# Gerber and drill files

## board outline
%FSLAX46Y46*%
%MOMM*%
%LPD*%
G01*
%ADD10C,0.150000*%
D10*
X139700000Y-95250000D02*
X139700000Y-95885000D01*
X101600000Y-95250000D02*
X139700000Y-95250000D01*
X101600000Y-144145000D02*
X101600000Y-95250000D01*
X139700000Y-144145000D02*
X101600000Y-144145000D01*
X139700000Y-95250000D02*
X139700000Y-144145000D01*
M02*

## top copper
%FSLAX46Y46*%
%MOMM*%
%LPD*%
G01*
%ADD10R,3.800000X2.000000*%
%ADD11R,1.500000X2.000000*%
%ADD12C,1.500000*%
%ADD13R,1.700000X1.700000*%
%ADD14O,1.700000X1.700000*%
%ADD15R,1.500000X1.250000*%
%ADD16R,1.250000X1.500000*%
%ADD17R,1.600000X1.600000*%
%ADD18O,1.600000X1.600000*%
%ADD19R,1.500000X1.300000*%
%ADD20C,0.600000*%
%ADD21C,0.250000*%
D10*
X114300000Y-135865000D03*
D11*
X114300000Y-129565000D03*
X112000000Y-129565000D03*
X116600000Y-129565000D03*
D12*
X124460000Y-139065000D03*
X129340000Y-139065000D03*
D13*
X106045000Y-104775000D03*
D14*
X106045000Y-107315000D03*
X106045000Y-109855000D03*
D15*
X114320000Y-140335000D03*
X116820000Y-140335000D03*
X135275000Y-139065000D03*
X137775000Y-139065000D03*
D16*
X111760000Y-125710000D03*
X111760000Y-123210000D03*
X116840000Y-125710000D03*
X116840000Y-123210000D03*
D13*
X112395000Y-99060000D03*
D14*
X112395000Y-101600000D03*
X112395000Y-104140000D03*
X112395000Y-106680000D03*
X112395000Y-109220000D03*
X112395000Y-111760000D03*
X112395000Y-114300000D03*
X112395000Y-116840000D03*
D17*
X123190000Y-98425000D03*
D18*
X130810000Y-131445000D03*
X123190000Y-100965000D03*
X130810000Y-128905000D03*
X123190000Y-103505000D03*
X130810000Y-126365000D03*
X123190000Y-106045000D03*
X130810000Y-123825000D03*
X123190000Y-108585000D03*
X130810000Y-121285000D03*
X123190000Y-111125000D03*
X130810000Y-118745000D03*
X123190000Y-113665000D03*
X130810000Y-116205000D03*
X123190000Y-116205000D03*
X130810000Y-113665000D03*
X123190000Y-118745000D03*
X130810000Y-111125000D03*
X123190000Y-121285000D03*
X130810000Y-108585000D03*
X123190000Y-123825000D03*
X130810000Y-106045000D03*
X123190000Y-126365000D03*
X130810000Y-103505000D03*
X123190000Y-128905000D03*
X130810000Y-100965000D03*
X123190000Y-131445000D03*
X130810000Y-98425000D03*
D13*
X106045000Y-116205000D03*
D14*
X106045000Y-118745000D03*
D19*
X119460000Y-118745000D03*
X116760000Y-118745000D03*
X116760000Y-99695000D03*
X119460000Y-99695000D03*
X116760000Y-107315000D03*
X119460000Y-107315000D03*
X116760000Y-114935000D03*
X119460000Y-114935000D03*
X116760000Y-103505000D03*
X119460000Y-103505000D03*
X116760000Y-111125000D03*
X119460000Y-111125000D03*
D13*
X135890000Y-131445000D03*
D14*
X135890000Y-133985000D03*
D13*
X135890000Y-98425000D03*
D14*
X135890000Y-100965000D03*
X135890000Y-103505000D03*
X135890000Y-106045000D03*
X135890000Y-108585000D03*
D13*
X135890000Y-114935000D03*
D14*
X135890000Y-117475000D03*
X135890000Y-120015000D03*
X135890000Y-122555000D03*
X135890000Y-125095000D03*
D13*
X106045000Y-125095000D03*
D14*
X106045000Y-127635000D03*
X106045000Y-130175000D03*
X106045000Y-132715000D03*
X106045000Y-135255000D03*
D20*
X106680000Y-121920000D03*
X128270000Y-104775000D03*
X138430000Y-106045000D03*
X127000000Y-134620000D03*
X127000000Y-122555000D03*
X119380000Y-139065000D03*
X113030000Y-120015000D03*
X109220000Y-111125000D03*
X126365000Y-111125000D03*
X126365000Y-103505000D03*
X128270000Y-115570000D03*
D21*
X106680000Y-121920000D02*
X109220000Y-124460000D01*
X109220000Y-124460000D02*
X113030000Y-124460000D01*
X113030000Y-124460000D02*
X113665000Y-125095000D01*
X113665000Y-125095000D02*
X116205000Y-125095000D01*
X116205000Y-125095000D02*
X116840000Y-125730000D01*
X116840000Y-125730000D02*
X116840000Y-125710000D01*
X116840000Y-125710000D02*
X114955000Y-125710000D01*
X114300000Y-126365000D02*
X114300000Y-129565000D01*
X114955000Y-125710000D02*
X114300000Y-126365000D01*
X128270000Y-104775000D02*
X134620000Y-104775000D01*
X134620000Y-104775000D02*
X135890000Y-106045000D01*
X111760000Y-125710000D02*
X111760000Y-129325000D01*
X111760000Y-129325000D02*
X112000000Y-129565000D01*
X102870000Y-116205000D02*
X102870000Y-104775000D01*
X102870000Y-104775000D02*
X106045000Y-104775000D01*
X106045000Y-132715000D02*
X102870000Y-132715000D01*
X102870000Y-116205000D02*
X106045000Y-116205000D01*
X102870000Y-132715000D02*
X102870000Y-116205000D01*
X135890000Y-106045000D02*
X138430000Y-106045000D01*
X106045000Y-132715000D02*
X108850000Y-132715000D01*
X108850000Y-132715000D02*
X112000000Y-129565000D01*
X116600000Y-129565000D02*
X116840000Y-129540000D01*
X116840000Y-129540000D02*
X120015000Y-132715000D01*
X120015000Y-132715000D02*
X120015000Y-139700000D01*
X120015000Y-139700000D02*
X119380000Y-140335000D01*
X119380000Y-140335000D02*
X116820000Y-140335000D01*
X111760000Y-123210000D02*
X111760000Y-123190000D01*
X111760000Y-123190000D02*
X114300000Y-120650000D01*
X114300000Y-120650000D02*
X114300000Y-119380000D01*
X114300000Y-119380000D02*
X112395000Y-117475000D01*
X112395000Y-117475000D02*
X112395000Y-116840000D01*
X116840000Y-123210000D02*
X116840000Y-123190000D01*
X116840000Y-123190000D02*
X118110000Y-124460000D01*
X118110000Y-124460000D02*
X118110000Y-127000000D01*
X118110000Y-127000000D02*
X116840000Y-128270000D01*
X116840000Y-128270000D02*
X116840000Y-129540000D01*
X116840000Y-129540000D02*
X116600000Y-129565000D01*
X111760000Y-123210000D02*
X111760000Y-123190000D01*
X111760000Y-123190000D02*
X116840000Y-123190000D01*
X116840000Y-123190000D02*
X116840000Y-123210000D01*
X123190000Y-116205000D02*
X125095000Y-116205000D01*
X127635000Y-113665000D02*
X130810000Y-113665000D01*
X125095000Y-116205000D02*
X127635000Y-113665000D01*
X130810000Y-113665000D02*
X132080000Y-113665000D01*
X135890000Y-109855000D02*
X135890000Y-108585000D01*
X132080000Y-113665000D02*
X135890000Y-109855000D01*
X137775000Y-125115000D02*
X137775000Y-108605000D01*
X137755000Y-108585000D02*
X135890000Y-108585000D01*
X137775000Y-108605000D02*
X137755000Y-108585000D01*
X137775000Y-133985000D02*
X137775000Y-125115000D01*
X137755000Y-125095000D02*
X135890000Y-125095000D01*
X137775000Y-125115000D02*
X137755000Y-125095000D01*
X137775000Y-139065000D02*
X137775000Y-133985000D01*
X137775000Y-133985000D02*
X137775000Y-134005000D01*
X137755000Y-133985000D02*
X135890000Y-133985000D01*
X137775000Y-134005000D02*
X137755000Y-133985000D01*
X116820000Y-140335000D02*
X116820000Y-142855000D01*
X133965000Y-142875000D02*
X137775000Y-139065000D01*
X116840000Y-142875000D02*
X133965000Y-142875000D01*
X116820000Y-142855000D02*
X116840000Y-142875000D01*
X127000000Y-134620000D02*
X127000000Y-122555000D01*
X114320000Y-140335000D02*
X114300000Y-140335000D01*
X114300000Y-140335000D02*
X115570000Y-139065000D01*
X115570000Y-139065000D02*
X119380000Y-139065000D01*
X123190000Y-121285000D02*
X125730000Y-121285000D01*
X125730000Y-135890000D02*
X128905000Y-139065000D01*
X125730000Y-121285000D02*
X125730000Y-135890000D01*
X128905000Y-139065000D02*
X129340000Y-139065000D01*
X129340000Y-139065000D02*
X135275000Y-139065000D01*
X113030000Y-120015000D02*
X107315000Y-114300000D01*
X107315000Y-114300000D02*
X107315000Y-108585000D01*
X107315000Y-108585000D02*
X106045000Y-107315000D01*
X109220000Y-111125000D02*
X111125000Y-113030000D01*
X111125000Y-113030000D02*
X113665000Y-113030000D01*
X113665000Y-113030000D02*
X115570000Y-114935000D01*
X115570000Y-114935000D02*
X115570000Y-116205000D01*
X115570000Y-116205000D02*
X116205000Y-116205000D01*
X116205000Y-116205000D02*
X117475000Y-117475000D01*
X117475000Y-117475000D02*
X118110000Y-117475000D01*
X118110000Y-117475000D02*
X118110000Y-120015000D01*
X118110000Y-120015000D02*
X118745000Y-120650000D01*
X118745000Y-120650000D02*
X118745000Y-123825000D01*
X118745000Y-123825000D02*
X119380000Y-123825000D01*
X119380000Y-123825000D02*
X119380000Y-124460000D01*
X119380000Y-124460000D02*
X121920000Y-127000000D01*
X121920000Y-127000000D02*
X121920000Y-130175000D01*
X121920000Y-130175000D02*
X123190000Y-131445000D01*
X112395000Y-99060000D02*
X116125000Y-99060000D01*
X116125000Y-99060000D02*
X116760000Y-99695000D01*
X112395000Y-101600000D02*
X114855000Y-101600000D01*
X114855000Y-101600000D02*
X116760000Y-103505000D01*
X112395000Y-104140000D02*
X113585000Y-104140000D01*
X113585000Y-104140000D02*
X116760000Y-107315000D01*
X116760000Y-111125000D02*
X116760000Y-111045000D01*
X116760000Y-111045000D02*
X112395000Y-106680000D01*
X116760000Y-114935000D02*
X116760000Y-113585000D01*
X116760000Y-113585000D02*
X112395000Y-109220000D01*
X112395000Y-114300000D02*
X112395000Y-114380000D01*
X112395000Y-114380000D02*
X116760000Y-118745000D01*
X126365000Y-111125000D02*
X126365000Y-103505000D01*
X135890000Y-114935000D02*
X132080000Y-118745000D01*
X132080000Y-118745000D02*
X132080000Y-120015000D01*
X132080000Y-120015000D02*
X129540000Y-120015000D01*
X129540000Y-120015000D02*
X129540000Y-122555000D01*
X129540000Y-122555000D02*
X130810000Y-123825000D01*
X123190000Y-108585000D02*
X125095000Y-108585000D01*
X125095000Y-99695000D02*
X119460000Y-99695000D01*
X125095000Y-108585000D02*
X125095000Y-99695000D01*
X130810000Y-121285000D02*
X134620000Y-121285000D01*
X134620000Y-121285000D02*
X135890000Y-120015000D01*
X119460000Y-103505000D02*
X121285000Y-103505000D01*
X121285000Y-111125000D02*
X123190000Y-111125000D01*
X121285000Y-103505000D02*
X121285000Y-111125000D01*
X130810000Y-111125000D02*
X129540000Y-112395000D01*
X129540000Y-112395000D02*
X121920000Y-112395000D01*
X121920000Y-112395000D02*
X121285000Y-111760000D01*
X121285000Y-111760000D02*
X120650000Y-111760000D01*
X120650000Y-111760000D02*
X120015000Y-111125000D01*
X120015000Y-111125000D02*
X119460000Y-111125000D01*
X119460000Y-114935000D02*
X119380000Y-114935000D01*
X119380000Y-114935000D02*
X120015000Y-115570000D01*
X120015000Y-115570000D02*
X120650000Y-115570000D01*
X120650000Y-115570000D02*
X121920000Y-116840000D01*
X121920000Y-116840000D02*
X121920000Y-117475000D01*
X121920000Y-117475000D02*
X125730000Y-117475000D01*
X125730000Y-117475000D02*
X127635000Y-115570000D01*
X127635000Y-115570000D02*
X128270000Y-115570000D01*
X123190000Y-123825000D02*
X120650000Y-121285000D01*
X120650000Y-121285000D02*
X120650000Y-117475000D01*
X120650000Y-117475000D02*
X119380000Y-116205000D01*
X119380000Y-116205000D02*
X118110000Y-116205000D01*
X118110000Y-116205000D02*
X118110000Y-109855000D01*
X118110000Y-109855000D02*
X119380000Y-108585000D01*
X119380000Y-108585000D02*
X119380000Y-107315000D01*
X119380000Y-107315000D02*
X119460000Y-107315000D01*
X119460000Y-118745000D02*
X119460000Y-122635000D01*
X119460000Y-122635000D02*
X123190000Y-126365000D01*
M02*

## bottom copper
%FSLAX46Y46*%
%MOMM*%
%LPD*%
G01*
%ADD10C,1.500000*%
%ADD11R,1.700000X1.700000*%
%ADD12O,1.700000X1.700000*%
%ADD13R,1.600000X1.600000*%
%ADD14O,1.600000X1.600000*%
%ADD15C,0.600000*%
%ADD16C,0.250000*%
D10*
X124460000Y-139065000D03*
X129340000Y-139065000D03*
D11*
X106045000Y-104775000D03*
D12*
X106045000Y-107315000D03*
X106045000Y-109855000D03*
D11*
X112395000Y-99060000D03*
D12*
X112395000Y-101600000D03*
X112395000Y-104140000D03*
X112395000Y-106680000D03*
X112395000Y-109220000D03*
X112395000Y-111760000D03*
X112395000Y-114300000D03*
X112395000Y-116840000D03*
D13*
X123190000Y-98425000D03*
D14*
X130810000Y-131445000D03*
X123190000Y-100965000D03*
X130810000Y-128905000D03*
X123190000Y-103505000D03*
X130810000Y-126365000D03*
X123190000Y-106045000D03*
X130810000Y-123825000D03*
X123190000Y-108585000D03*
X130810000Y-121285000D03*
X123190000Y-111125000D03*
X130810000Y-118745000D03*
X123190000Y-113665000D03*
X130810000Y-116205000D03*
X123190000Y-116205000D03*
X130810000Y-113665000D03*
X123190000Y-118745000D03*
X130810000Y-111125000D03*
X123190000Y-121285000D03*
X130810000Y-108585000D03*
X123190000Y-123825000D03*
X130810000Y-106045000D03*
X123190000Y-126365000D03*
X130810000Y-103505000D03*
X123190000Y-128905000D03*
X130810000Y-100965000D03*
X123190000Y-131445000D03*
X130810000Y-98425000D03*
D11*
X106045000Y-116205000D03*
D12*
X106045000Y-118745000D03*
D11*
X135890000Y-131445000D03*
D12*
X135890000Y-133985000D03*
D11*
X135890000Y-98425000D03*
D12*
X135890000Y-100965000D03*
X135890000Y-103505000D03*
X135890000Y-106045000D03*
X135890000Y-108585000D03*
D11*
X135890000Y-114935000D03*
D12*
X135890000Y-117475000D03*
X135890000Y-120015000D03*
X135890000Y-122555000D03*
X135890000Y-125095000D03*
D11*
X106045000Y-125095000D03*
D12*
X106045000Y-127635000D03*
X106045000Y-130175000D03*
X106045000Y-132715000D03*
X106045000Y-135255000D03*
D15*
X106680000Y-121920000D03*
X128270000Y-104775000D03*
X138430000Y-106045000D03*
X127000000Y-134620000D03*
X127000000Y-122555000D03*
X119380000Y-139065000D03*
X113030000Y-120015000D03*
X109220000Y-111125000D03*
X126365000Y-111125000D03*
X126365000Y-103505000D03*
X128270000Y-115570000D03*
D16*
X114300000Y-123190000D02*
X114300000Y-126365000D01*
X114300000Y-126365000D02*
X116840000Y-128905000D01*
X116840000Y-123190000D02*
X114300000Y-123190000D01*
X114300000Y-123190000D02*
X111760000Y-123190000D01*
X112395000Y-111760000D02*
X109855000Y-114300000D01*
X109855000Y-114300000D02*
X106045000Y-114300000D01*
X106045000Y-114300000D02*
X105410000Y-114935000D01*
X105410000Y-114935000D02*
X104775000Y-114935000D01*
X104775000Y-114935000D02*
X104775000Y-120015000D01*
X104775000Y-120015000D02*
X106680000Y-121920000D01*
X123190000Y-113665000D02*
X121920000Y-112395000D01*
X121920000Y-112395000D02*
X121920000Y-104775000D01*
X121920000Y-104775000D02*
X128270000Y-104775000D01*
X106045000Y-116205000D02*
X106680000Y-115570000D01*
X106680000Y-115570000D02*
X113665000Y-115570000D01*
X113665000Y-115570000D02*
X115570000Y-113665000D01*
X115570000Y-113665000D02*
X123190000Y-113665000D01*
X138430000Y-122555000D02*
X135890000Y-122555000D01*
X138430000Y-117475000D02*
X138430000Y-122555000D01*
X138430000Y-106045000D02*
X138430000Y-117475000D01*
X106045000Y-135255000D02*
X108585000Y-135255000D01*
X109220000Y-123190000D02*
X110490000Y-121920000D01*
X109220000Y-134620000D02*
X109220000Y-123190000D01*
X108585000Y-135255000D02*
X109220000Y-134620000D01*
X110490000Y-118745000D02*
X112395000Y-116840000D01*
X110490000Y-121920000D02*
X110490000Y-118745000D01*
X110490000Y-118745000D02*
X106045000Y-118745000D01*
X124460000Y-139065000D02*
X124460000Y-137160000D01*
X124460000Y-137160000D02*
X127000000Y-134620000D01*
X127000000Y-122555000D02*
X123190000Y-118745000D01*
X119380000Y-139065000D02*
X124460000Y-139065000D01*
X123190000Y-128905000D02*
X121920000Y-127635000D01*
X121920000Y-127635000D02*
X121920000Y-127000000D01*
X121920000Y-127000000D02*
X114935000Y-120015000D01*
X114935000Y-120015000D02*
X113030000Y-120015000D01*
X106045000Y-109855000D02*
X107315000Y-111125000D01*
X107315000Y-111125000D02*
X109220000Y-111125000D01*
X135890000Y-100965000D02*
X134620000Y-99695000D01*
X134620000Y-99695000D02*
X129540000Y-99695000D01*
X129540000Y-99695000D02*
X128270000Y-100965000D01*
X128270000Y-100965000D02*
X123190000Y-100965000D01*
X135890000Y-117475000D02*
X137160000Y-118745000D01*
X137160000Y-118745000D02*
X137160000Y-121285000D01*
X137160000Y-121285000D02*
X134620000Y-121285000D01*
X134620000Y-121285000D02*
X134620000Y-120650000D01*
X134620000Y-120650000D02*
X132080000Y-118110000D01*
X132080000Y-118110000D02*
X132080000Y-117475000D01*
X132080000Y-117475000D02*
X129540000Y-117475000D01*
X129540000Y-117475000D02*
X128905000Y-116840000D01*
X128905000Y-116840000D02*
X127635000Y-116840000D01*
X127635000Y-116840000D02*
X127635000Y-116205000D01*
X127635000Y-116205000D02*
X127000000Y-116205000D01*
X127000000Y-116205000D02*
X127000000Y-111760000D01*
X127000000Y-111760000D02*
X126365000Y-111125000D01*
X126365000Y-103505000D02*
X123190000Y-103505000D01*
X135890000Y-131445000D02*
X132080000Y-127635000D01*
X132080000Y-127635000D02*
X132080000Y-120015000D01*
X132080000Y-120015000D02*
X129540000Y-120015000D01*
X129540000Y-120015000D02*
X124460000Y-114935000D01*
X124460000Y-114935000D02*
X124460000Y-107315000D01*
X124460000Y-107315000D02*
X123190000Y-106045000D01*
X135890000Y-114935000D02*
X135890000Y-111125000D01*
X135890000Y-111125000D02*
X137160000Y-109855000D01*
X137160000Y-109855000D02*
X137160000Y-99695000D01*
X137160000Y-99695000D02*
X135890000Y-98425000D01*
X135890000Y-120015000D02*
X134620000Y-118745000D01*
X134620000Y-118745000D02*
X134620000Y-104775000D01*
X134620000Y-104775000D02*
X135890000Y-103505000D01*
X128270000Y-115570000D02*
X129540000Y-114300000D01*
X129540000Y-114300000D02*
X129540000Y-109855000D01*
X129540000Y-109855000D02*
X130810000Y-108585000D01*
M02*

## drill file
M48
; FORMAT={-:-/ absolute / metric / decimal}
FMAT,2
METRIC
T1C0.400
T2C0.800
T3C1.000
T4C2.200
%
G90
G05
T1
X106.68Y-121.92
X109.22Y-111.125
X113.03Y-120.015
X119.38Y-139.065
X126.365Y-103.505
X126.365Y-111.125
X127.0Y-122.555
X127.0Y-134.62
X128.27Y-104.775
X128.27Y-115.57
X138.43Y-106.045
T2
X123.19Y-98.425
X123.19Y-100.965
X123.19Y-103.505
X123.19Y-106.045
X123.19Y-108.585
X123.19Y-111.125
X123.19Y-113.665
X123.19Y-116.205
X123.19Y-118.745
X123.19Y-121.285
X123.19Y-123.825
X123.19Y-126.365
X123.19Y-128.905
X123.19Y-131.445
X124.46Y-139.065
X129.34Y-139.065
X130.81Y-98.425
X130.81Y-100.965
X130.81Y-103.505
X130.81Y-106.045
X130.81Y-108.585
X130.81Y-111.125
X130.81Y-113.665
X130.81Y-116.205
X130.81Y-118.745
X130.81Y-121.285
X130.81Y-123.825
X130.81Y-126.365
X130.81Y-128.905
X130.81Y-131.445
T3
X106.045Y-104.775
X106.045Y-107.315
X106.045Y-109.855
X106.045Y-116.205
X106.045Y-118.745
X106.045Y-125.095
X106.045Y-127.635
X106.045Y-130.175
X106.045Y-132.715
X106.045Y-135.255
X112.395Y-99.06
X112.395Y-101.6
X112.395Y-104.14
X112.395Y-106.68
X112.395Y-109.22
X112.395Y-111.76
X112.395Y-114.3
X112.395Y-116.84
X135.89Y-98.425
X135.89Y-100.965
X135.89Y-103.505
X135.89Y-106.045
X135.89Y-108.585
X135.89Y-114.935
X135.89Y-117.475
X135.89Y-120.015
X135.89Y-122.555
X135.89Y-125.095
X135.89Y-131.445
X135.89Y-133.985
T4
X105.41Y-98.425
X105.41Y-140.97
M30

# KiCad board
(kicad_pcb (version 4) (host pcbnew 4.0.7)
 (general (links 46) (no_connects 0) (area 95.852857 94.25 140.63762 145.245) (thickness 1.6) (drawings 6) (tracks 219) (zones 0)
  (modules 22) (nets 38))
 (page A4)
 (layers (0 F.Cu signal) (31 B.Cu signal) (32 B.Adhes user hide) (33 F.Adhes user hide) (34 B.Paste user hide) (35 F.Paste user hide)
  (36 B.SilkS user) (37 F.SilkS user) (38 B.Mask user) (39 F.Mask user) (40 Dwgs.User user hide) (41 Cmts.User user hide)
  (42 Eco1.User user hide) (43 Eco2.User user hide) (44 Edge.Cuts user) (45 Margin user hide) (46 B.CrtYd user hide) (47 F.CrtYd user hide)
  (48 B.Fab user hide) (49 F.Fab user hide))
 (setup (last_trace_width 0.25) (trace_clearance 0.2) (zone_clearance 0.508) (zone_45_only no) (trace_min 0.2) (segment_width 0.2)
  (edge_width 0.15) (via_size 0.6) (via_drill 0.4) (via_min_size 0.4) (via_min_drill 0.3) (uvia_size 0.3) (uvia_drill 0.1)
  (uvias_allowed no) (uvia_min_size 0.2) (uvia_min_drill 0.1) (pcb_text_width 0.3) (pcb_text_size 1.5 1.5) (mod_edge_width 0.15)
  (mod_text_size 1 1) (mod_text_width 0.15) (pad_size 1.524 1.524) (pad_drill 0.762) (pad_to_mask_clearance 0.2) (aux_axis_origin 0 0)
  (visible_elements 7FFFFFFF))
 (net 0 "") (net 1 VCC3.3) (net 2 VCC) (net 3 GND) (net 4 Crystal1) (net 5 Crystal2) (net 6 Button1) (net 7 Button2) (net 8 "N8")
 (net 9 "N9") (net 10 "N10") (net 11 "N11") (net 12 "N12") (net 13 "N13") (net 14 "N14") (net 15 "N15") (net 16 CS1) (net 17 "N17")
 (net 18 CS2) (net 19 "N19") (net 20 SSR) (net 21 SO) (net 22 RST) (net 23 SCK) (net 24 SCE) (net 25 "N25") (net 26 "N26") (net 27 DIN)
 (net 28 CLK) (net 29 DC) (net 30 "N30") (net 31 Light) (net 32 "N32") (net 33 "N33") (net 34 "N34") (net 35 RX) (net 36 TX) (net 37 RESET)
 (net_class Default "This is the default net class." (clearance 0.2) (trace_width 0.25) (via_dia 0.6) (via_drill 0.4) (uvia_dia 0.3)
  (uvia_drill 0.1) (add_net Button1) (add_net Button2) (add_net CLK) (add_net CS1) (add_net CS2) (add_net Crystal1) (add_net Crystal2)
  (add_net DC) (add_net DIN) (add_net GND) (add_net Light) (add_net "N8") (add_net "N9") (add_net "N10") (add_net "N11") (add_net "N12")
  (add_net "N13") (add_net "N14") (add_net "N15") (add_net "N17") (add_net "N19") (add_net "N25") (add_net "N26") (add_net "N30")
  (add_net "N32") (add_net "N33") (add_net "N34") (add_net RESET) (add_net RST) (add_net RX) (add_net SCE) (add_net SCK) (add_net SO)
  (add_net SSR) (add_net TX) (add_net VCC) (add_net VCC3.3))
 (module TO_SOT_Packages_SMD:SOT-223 (layer F.Cu) (at 114.3 132.715 270)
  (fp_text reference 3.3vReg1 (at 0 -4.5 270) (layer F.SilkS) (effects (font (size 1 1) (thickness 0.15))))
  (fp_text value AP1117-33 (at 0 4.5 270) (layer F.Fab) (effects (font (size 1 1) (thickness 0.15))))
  (pad 4 smd rect (at 3.15 0 270) (size 2 3.8) (layers F.Cu F.Paste F.Mask))
  (pad 2 smd rect (at -3.15 0 270) (size 2 1.5) (layers F.Cu F.Paste F.Mask) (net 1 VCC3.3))
  (pad 3 smd rect (at -3.15 2.3 270) (size 2 1.5) (layers F.Cu F.Paste F.Mask) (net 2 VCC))
  (pad 1 smd rect (at -3.15 -2.3 270) (size 2 1.5) (layers F.Cu F.Paste F.Mask) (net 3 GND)))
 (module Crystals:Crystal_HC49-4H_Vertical (layer F.Cu) (at 124.46 139.065)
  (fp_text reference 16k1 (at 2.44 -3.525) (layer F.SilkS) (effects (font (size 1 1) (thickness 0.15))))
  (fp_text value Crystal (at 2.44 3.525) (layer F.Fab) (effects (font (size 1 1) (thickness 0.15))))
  (pad 1 thru_hole circle (at 0 0) (size 1.5 1.5) (drill 0.8) (layers *.Cu *.Mask) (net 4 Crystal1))
  (pad 2 thru_hole circle (at 4.88 0) (size 1.5 1.5) (drill 0.8) (layers *.Cu *.Mask) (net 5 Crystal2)))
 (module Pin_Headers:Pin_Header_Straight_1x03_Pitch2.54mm (layer F.Cu) (at 106.045 104.775)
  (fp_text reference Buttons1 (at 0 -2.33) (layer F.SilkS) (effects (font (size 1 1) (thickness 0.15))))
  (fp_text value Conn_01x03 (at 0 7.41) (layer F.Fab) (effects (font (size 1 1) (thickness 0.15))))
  (pad 1 thru_hole rect (at 0 0) (size 1.7 1.7) (drill 1) (layers *.Cu *.Mask) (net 2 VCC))
  (pad 2 thru_hole oval (at 0 2.54) (size 1.7 1.7) (drill 1) (layers *.Cu *.Mask) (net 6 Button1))
  (pad 3 thru_hole oval (at 0 5.08) (size 1.7 1.7) (drill 1) (layers *.Cu *.Mask) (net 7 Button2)))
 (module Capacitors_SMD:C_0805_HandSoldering (layer F.Cu) (at 115.57 140.335)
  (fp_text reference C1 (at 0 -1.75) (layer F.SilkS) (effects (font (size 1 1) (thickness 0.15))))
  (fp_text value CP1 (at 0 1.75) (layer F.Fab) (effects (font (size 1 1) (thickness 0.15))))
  (pad 1 smd rect (at -1.25 0) (size 1.5 1.25) (layers F.Cu F.Paste F.Mask) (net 4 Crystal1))
  (pad 2 smd rect (at 1.25 0) (size 1.5 1.25) (layers F.Cu F.Paste F.Mask) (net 3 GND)))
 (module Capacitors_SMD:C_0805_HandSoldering (layer F.Cu) (at 136.525 139.065)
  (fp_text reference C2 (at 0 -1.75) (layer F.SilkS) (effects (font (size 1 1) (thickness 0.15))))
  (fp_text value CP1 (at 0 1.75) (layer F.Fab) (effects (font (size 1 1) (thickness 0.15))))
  (pad 1 smd rect (at -1.25 0) (size 1.5 1.25) (layers F.Cu F.Paste F.Mask) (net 5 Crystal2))
  (pad 2 smd rect (at 1.25 0) (size 1.5 1.25) (layers F.Cu F.Paste F.Mask) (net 3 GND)))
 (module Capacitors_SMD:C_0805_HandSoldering (layer F.Cu) (at 111.76 124.46 90)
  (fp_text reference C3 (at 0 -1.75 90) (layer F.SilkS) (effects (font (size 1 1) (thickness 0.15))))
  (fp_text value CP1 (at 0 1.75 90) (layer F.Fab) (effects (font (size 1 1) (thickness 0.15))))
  (pad 1 smd rect (at -1.25 0 90) (size 1.5 1.25) (layers F.Cu F.Paste F.Mask) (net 2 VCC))
  (pad 2 smd rect (at 1.25 0 90) (size 1.5 1.25) (layers F.Cu F.Paste F.Mask) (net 3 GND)))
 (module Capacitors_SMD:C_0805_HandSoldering (layer F.Cu) (at 116.84 124.46 90)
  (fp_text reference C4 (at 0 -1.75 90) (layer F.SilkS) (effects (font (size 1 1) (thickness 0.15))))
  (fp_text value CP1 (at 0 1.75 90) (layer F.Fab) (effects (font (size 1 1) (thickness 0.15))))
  (pad 1 smd rect (at -1.25 0 90) (size 1.5 1.25) (layers F.Cu F.Paste F.Mask) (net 1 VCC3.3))
  (pad 2 smd rect (at 1.25 0 90) (size 1.5 1.25) (layers F.Cu F.Paste F.Mask) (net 3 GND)))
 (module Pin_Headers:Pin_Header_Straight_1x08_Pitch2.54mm (layer F.Cu) (at 112.395 99.06)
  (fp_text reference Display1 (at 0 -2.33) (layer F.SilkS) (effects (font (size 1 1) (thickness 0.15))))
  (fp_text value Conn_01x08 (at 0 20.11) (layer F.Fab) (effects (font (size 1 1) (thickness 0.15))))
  (pad 1 thru_hole rect (at 0 0) (size 1.7 1.7) (drill 1) (layers *.Cu *.Mask) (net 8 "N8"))
  (pad 2 thru_hole oval (at 0 2.54) (size 1.7 1.7) (drill 1) (layers *.Cu *.Mask) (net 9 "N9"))
  (pad 3 thru_hole oval (at 0 5.08) (size 1.7 1.7) (drill 1) (layers *.Cu *.Mask) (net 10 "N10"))
  (pad 4 thru_hole oval (at 0 7.62) (size 1.7 1.7) (drill 1) (layers *.Cu *.Mask) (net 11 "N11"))
  (pad 5 thru_hole oval (at 0 10.16) (size 1.7 1.7) (drill 1) (layers *.Cu *.Mask) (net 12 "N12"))
  (pad 6 thru_hole oval (at 0 12.7) (size 1.7 1.7) (drill 1) (layers *.Cu *.Mask) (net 1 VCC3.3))
  (pad 7 thru_hole oval (at 0 15.24) (size 1.7 1.7) (drill 1) (layers *.Cu *.Mask) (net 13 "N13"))
  (pad 8 thru_hole oval (at 0 17.78) (size 1.7 1.7) (drill 1) (layers *.Cu *.Mask) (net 3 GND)))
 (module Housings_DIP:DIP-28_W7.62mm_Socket (layer F.Cu) (at 123.19 98.425)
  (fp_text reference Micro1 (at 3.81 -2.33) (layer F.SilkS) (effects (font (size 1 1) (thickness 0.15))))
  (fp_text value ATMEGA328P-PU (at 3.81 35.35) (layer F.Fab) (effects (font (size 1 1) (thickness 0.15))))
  (pad 1 thru_hole rect (at 0 0) (size 1.6 1.6) (drill 0.8) (layers *.Cu *.Mask) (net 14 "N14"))
  (pad 15 thru_hole oval (at 7.62 33.02) (size 1.6 1.6) (drill 0.8) (layers *.Cu *.Mask) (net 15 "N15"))
  (pad 2 thru_hole oval (at 0 2.54) (size 1.6 1.6) (drill 0.8) (layers *.Cu *.Mask) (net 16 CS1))
  (pad 16 thru_hole oval (at 7.62 30.48) (size 1.6 1.6) (drill 0.8) (layers *.Cu *.Mask) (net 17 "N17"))
  (pad 3 thru_hole oval (at 0 5.08) (size 1.6 1.6) (drill 0.8) (layers *.Cu *.Mask) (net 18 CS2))
  (pad 17 thru_hole oval (at 7.62 27.94) (size 1.6 1.6) (drill 0.8) (layers *.Cu *.Mask) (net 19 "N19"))
  (pad 4 thru_hole oval (at 0 7.62) (size 1.6 1.6) (drill 0.8) (layers *.Cu *.Mask) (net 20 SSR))
  (pad 18 thru_hole oval (at 7.62 25.4) (size 1.6 1.6) (drill 0.8) (layers *.Cu *.Mask) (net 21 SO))
  (pad 5 thru_hole oval (at 0 10.16) (size 1.6 1.6) (drill 0.8) (layers *.Cu *.Mask) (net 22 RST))
  (pad 19 thru_hole oval (at 7.62 22.86) (size 1.6 1.6) (drill 0.8) (layers *.Cu *.Mask) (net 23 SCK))
  (pad 6 thru_hole oval (at 0 12.7) (size 1.6 1.6) (drill 0.8) (layers *.Cu *.Mask) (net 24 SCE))
  (pad 20 thru_hole oval (at 7.62 20.32) (size 1.6 1.6) (drill 0.8) (layers *.Cu *.Mask) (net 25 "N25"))
  (pad 7 thru_hole oval (at 0 15.24) (size 1.6 1.6) (drill 0.8) (layers *.Cu *.Mask) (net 2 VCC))
  (pad 21 thru_hole oval (at 7.62 17.78) (size 1.6 1.6) (drill 0.8) (layers *.Cu *.Mask) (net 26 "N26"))
  (pad 8 thru_hole oval (at 0 17.78) (size 1.6 1.6) (drill 0.8) (layers *.Cu *.Mask) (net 3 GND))
  (pad 22 thru_hole oval (at 7.62 15.24) (size 1.6 1.6) (drill 0.8) (layers *.Cu *.Mask) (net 3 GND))
  (pad 9 thru_hole oval (at 0 20.32) (size 1.6 1.6) (drill 0.8) (layers *.Cu *.Mask) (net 4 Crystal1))
  (pad 23 thru_hole oval (at 7.62 12.7) (size 1.6 1.6) (drill 0.8) (layers *.Cu *.Mask) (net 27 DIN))
  (pad 10 thru_hole oval (at 0 22.86) (size 1.6 1.6) (drill 0.8) (layers *.Cu *.Mask) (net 5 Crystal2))
  (pad 24 thru_hole oval (at 7.62 10.16) (size 1.6 1.6) (drill 0.8) (layers *.Cu *.Mask) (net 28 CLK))
  (pad 11 thru_hole oval (at 0 25.4) (size 1.6 1.6) (drill 0.8) (layers *.Cu *.Mask) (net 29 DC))
  (pad 25 thru_hole oval (at 7.62 7.62) (size 1.6 1.6) (drill 0.8) (layers *.Cu *.Mask) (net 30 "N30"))
  (pad 12 thru_hole oval (at 0 27.94) (size 1.6 1.6) (drill 0.8) (layers *.Cu *.Mask) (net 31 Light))
  (pad 26 thru_hole oval (at 7.62 5.08) (size 1.6 1.6) (drill 0.8) (layers *.Cu *.Mask) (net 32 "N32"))
  (pad 13 thru_hole oval (at 0 30.48) (size 1.6 1.6) (drill 0.8) (layers *.Cu *.Mask) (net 6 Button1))
  (pad 27 thru_hole oval (at 7.62 2.54) (size 1.6 1.6) (drill 0.8) (layers *.Cu *.Mask) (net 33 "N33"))
  (pad 14 thru_hole oval (at 0 33.02) (size 1.6 1.6) (drill 0.8) (layers *.Cu *.Mask) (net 7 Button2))
  (pad 28 thru_hole oval (at 7.62 0) (size 1.6 1.6) (drill 0.8) (layers *.Cu *.Mask) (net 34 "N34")))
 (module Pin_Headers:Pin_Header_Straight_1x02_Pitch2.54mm (layer F.Cu) (at 106.045 116.205)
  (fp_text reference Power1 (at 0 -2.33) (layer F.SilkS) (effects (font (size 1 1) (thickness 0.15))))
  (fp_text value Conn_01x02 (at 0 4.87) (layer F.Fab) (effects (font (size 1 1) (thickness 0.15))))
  (pad 1 thru_hole rect (at 0 0) (size 1.7 1.7) (drill 1) (layers *.Cu *.Mask) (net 2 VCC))
  (pad 2 thru_hole oval (at 0 2.54) (size 1.7 1.7) (drill 1) (layers *.Cu *.Mask) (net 3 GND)))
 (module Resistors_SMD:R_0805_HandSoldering (layer F.Cu) (at 118.11 118.745 180)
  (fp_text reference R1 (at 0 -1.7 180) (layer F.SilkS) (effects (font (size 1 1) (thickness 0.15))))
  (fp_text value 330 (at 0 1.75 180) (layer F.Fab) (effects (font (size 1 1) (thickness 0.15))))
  (pad 1 smd rect (at -1.35 0 180) (size 1.5 1.3) (layers F.Cu F.Paste F.Mask) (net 31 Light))
  (pad 2 smd rect (at 1.35 0 180) (size 1.5 1.3) (layers F.Cu F.Paste F.Mask) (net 13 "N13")))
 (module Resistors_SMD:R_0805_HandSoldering (layer F.Cu) (at 118.11 99.695)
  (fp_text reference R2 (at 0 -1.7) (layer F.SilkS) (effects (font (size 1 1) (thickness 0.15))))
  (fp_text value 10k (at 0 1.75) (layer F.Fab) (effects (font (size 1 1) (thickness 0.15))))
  (pad 1 smd rect (at -1.35 0) (size 1.5 1.3) (layers F.Cu F.Paste F.Mask) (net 8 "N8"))
  (pad 2 smd rect (at 1.35 0) (size 1.5 1.3) (layers F.Cu F.Paste F.Mask) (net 22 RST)))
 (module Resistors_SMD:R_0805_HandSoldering (layer F.Cu) (at 118.11 107.315)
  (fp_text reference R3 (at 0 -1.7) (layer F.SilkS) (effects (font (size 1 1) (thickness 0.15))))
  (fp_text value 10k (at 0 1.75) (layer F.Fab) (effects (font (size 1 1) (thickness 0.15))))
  (pad 1 smd rect (at -1.35 0) (size 1.5 1.3) (layers F.Cu F.Paste F.Mask) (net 10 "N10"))
  (pad 2 smd rect (at 1.35 0) (size 1.5 1.3) (layers F.Cu F.Paste F.Mask) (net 29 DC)))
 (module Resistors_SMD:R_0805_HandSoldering (layer F.Cu) (at 118.11 114.935)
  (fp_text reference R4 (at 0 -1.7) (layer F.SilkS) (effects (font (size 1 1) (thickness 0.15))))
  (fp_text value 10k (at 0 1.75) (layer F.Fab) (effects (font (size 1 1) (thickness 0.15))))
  (pad 1 smd rect (at -1.35 0) (size 1.5 1.3) (layers F.Cu F.Paste F.Mask) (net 12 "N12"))
  (pad 2 smd rect (at 1.35 0) (size 1.5 1.3) (layers F.Cu F.Paste F.Mask) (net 28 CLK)))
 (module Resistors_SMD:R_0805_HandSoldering (layer F.Cu) (at 118.11 103.505)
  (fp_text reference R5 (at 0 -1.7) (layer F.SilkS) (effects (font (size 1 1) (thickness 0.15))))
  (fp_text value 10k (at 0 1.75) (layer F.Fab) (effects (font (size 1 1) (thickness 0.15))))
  (pad 1 smd rect (at -1.35 0) (size 1.5 1.3) (layers F.Cu F.Paste F.Mask) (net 9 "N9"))
  (pad 2 smd rect (at 1.35 0) (size 1.5 1.3) (layers F.Cu F.Paste F.Mask) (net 24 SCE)))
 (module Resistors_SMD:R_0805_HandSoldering (layer F.Cu) (at 118.11 111.125)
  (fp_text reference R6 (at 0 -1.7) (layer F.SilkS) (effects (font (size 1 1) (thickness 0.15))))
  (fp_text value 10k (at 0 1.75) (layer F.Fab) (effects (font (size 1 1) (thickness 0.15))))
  (pad 1 smd rect (at -1.35 0) (size 1.5 1.3) (layers F.Cu F.Paste F.Mask) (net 11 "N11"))
  (pad 2 smd rect (at 1.35 0) (size 1.5 1.3) (layers F.Cu F.Paste F.Mask) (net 27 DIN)))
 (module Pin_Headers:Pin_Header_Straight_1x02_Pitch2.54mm (layer F.Cu) (at 135.89 131.445)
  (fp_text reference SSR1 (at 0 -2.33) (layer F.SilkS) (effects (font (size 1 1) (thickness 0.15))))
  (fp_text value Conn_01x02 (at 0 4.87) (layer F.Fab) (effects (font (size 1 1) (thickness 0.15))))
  (pad 1 thru_hole rect (at 0 0) (size 1.7 1.7) (drill 1) (layers *.Cu *.Mask) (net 20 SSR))
  (pad 2 thru_hole oval (at 0 2.54) (size 1.7 1.7) (drill 1) (layers *.Cu *.Mask) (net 3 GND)))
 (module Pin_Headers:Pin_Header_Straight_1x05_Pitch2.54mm (layer F.Cu) (at 135.89 98.425)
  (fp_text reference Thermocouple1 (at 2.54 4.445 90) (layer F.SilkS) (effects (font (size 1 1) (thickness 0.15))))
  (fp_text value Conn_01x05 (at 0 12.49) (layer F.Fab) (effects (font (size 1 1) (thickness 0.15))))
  (pad 1 thru_hole rect (at 0 0) (size 1.7 1.7) (drill 1) (layers *.Cu *.Mask) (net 21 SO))
  (pad 2 thru_hole oval (at 0 2.54) (size 1.7 1.7) (drill 1) (layers *.Cu *.Mask) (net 16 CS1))
  (pad 3 thru_hole oval (at 0 5.08) (size 1.7 1.7) (drill 1) (layers *.Cu *.Mask) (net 23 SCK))
  (pad 4 thru_hole oval (at 0 7.62) (size 1.7 1.7) (drill 1) (layers *.Cu *.Mask) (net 2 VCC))
  (pad 5 thru_hole oval (at 0 10.16) (size 1.7 1.7) (drill 1) (layers *.Cu *.Mask) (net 3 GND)))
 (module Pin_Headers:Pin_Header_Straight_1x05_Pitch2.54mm (layer F.Cu) (at 135.89 114.935)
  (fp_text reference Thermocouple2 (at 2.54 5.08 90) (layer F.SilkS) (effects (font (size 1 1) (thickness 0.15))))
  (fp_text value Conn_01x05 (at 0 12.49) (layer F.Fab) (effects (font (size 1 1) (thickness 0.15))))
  (pad 1 thru_hole rect (at 0 0) (size 1.7 1.7) (drill 1) (layers *.Cu *.Mask) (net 21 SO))
  (pad 2 thru_hole oval (at 0 2.54) (size 1.7 1.7) (drill 1) (layers *.Cu *.Mask) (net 18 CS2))
  (pad 3 thru_hole oval (at 0 5.08) (size 1.7 1.7) (drill 1) (layers *.Cu *.Mask) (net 23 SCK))
  (pad 4 thru_hole oval (at 0 7.62) (size 1.7 1.7) (drill 1) (layers *.Cu *.Mask) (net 2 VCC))
  (pad 5 thru_hole oval (at 0 10.16) (size 1.7 1.7) (drill 1) (layers *.Cu *.Mask) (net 3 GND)))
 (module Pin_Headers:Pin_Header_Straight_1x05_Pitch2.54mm (layer F.Cu) (at 106.045 125.095)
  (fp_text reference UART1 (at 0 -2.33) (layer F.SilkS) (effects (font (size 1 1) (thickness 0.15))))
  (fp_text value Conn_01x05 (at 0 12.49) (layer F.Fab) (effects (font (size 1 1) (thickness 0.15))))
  (pad 1 thru_hole rect (at 0 0) (size 1.7 1.7) (drill 1) (layers *.Cu *.Mask) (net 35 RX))
  (pad 2 thru_hole oval (at 0 2.54) (size 1.7 1.7) (drill 1) (layers *.Cu *.Mask) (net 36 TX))
  (pad 3 thru_hole oval (at 0 5.08) (size 1.7 1.7) (drill 1) (layers *.Cu *.Mask) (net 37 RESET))
  (pad 4 thru_hole oval (at 0 7.62) (size 1.7 1.7) (drill 1) (layers *.Cu *.Mask) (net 2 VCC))
  (pad 5 thru_hole oval (at 0 10.16) (size 1.7 1.7) (drill 1) (layers *.Cu *.Mask) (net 3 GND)))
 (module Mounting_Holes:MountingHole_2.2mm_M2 (layer F.Cu) (at 105.41 98.425)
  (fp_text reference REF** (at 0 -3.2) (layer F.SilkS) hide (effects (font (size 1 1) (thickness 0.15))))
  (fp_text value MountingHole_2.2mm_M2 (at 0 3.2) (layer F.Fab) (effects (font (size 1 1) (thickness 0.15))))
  (pad 1 np_thru_hole circle (at 0 0) (size 2.2 2.2) (drill 2.2) (layers *.Cu *.Mask)))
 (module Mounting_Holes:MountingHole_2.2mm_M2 (layer F.Cu) (at 105.41 140.97)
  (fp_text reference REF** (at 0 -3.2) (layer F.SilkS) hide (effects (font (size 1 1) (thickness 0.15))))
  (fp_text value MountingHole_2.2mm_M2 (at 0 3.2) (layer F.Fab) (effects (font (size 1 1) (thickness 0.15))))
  (pad 1 np_thru_hole circle (at 0 0) (size 2.2 2.2) (drill 2.2) (layers *.Cu *.Mask)))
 (gr_line (start 139.7 95.25) (end 139.7 95.885) (angle 90) (layer Edge.Cuts) (width 0.15))
 (gr_line (start 101.6 95.25) (end 139.7 95.25) (angle 90) (layer Edge.Cuts) (width 0.15))
 (gr_line (start 101.6 144.145) (end 101.6 95.25) (angle 90) (layer Edge.Cuts) (width 0.15))
 (gr_line (start 139.7 144.145) (end 101.6 144.145) (angle 90) (layer Edge.Cuts) (width 0.15))
 (gr_line (start 139.7 95.25) (end 139.7 144.145) (angle 90) (layer Edge.Cuts) (width 0.15))
 (segment (start 114.3 123.19) (end 114.3 126.365) (width 0.25) (layer B.Cu) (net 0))
 (segment (start 114.3 126.365) (end 116.84 128.905) (width 0.25) (layer B.Cu) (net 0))
 (segment (start 116.84 123.19) (end 114.3 123.19) (width 0.25) (layer B.Cu) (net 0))
 (segment (start 114.3 123.19) (end 111.76 123.19) (width 0.25) (layer B.Cu) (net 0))
 (segment (start 112.395 111.76) (end 109.855 114.3) (width 0.25) (layer B.Cu) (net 1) (status 80000))
 (segment (start 109.855 114.3) (end 106.045 114.3) (width 0.25) (layer B.Cu) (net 1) (status 80000))
 (segment (start 106.045 114.3) (end 105.41 114.935) (width 0.25) (layer B.Cu) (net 1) (status 80000))
 (segment (start 105.41 114.935) (end 104.775 114.935) (width 0.25) (layer B.Cu) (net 1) (status 80000))
 (segment (start 104.775 114.935) (end 104.775 120.015) (width 0.25) (layer B.Cu) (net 1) (status 80000))
 (segment (start 104.775 120.015) (end 106.68 121.92) (width 0.25) (layer B.Cu) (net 1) (status 80000))
 (via (at 106.68 121.92) (size 0.6) (layers F.Cu B.Cu) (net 1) (status 80000))
 (segment (start 106.68 121.92) (end 109.22 124.46) (width 0.25) (layer F.Cu) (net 1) (status 80000))
 (segment (start 109.22 124.46) (end 113.03 124.46) (width 0.25) (layer F.Cu) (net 1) (status 80000))
 (segment (start 113.03 124.46) (end 113.665 125.095) (width 0.25) (layer F.Cu) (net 1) (status 80000))
 (segment (start 113.665 125.095) (end 116.205 125.095) (width 0.25) (layer F.Cu) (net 1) (status 80000))
 (segment (start 116.205 125.095) (end 116.84 125.73) (width 0.25) (layer F.Cu) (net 1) (status 80000))
 (segment (start 116.84 125.73) (end 116.84 125.71) (width 0.25) (layer F.Cu) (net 1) (status 80000))
 (segment (start 116.84 125.71) (end 114.955 125.71) (width 0.25) (layer F.Cu) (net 1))
 (segment (start 114.3 126.365) (end 114.3 129.565) (width 0.25) (layer F.Cu) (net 1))
 (segment (start 114.955 125.71) (end 114.3 126.365) (width 0.25) (layer F.Cu) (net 1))
 (segment (start 123.19 113.665) (end 121.92 112.395) (width 0.25) (layer B.Cu) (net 2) (status 80000))
 (segment (start 121.92 112.395) (end 121.92 104.775) (width 0.25) (layer B.Cu) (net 2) (status 80000))
 (segment (start 121.92 104.775) (end 128.27 104.775) (width 0.25) (layer B.Cu) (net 2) (status 80000))
 (via (at 128.27 104.775) (size 0.6) (layers F.Cu B.Cu) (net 2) (status 80000))
 (segment (start 128.27 104.775) (end 134.62 104.775) (width 0.25) (layer F.Cu) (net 2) (status 80000))
 (segment (start 134.62 104.775) (end 135.89 106.045) (width 0.25) (layer F.Cu) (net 2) (status 80000))
 (segment (start 111.76 125.71) (end 111.76 129.325) (width 0.25) (layer F.Cu) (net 2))
 (segment (start 111.76 129.325) (end 112 129.565) (width 0.25) (layer F.Cu) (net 2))
 (segment (start 106.045 116.205) (end 106.68 115.57) (width 0.25) (layer B.Cu) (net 2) (status 80000))
 (segment (start 106.68 115.57) (end 113.665 115.57) (width 0.25) (layer B.Cu) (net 2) (status 80000))
 (segment (start 113.665 115.57) (end 115.57 113.665) (width 0.25) (layer B.Cu) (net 2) (status 80000))
 (segment (start 115.57 113.665) (end 123.19 113.665) (width 0.25) (layer B.Cu) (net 2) (status 80000))
 (segment (start 102.87 116.205) (end 102.87 104.775) (width 0.25) (layer F.Cu) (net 2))
 (segment (start 102.87 104.775) (end 106.045 104.775) (width 0.25) (layer F.Cu) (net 2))
 (segment (start 106.045 132.715) (end 102.87 132.715) (width 0.25) (layer F.Cu) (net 2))
 (segment (start 102.87 116.205) (end 106.045 116.205) (width 0.25) (layer F.Cu) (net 2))
 (segment (start 102.87 132.715) (end 102.87 116.205) (width 0.25) (layer F.Cu) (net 2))
 (segment (start 135.89 106.045) (end 138.43 106.045) (width 0.25) (layer F.Cu) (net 2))
 (segment (start 138.43 122.555) (end 135.89 122.555) (width 0.25) (layer B.Cu) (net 2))
 (segment (start 138.43 117.475) (end 138.43 122.555) (width 0.25) (layer B.Cu) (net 2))
 (segment (start 138.43 106.045) (end 138.43 117.475) (width 0.25) (layer B.Cu) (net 2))
 (via (at 138.43 106.045) (size 0.6) (drill 0.4) (layers F.Cu B.Cu) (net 2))
 (segment (start 106.045 132.715) (end 108.85 132.715) (width 0.25) (layer F.Cu) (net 2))
 (segment (start 108.85 132.715) (end 112 129.565) (width 0.25) (layer F.Cu) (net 2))
 (segment (start 116.6 129.565) (end 116.84 129.54) (width 0.25) (layer F.Cu) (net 3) (status 80000))
 (segment (start 116.84 129.54) (end 120.015 132.715) (width 0.25) (layer F.Cu) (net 3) (status 80000))
 (segment (start 120.015 132.715) (end 120.015 139.7) (width 0.25) (layer F.Cu) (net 3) (status 80000))
 (segment (start 120.015 139.7) (end 119.38 140.335) (width 0.25) (layer F.Cu) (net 3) (status 80000))
 (segment (start 119.38 140.335) (end 116.82 140.335) (width 0.25) (layer F.Cu) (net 3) (status 80000))
 (segment (start 111.76 123.21) (end 111.76 123.19) (width 0.25) (layer F.Cu) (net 3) (status 80000))
 (segment (start 111.76 123.19) (end 114.3 120.65) (width 0.25) (layer F.Cu) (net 3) (status 80000))
 (segment (start 114.3 120.65) (end 114.3 119.38) (width 0.25) (layer F.Cu) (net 3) (status 80000))
 (segment (start 114.3 119.38) (end 112.395 117.475) (width 0.25) (layer F.Cu) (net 3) (status 80000))
 (segment (start 112.395 117.475) (end 112.395 116.84) (width 0.25) (layer F.Cu) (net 3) (status 80000))
 (segment (start 106.045 135.255) (end 108.585 135.255) (width 0.25) (layer B.Cu) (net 3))
 (segment (start 109.22 123.19) (end 110.49 121.92) (width 0.25) (layer B.Cu) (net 3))
 (segment (start 109.22 134.62) (end 109.22 123.19) (width 0.25) (layer B.Cu) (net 3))
 (segment (start 108.585 135.255) (end 109.22 134.62) (width 0.25) (layer B.Cu) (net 3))
 (segment (start 116.84 123.21) (end 116.84 123.19) (width 0.25) (layer F.Cu) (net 3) (status 80000))
 (segment (start 116.84 123.19) (end 118.11 124.46) (width 0.25) (layer F.Cu) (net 3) (status 80000))
 (segment (start 118.11 124.46) (end 118.11 127) (width 0.25) (layer F.Cu) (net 3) (status 80000))
 (segment (start 118.11 127) (end 116.84 128.27) (width 0.25) (layer F.Cu) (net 3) (status 80000))
 (segment (start 116.84 128.27) (end 116.84 129.54) (width 0.25) (layer F.Cu) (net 3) (status 80000))
 (segment (start 116.84 129.54) (end 116.6 129.565) (width 0.25) (layer F.Cu) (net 3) (status 80000))
 (segment (start 111.76 123.21) (end 111.76 123.19) (width 0.25) (layer F.Cu) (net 3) (status 80000))
 (segment (start 111.76 123.19) (end 116.84 123.19) (width 0.25) (layer F.Cu) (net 3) (status 80000))
 (segment (start 116.84 123.19) (end 116.84 123.21) (width 0.25) (layer F.Cu) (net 3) (status 80000))
 (segment (start 110.49 118.745) (end 112.395 116.84) (width 0.25) (layer B.Cu) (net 3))
 (segment (start 110.49 121.92) (end 110.49 118.745) (width 0.25) (layer B.Cu) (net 3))
 (segment (start 110.49 118.745) (end 106.045 118.745) (width 0.25) (layer B.Cu) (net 3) (status 80000))
 (segment (start 123.19 116.205) (end 125.095 116.205) (width 0.25) (layer F.Cu) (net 3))
 (segment (start 127.635 113.665) (end 130.81 113.665) (width 0.25) (layer F.Cu) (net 3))
 (segment (start 125.095 116.205) (end 127.635 113.665) (width 0.25) (layer F.Cu) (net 3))
 (segment (start 130.81 113.665) (end 132.08 113.665) (width 0.25) (layer F.Cu) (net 3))
 (segment (start 135.89 109.855) (end 135.89 108.585) (width 0.25) (layer F.Cu) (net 3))
 (segment (start 132.08 113.665) (end 135.89 109.855) (width 0.25) (layer F.Cu) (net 3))
 (segment (start 137.775 125.115) (end 137.775 108.605) (width 0.25) (layer F.Cu) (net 3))
 (segment (start 137.755 108.585) (end 135.89 108.585) (width 0.25) (layer F.Cu) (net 3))
 (segment (start 137.775 108.605) (end 137.755 108.585) (width 0.25) (layer F.Cu) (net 3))
 (segment (start 137.775 133.985) (end 137.775 125.115) (width 0.25) (layer F.Cu) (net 3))
 (segment (start 137.755 125.095) (end 135.89 125.095) (width 0.25) (layer F.Cu) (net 3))
 (segment (start 137.775 125.115) (end 137.755 125.095) (width 0.25) (layer F.Cu) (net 3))
 (segment (start 137.775 139.065) (end 137.775 133.985) (width 0.25) (layer F.Cu) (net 3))
 (segment (start 137.775 133.985) (end 137.775 134.005) (width 0.25) (layer F.Cu) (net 3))
 (segment (start 137.755 133.985) (end 135.89 133.985) (width 0.25) (layer F.Cu) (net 3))
 (segment (start 137.775 134.005) (end 137.755 133.985) (width 0.25) (layer F.Cu) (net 3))
 (segment (start 116.82 140.335) (end 116.82 142.855) (width 0.25) (layer F.Cu) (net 3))
 (segment (start 133.965 142.875) (end 137.775 139.065) (width 0.25) (layer F.Cu) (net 3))
 (segment (start 116.84 142.875) (end 133.965 142.875) (width 0.25) (layer F.Cu) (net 3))
 (segment (start 116.82 142.855) (end 116.84 142.875) (width 0.25) (layer F.Cu) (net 3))
 (segment (start 124.46 139.065) (end 124.46 137.16) (width 0.25) (layer B.Cu) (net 4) (status 80000))
 (segment (start 124.46 137.16) (end 127 134.62) (width 0.25) (layer B.Cu) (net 4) (status 80000))
 (via (at 127 134.62) (size 0.6) (layers F.Cu B.Cu) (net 4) (status 80000))
 (segment (start 127 134.62) (end 127 122.555) (width 0.25) (layer F.Cu) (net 4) (status 80000))
 (via (at 127 122.555) (size 0.6) (layers F.Cu B.Cu) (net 4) (status 80000))
 (segment (start 127 122.555) (end 123.19 118.745) (width 0.25) (layer B.Cu) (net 4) (status 80000))
 (segment (start 114.32 140.335) (end 114.3 140.335) (width 0.25) (layer F.Cu) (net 4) (status 80000))
 (segment (start 114.3 140.335) (end 115.57 139.065) (width 0.25) (layer F.Cu) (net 4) (status 80000))
 (segment (start 115.57 139.065) (end 119.38 139.065) (width 0.25) (layer F.Cu) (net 4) (status 80000))
 (via (at 119.38 139.065) (size 0.6) (layers F.Cu B.Cu) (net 4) (status 80000))
 (segment (start 119.38 139.065) (end 124.46 139.065) (width 0.25) (layer B.Cu) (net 4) (status 80000))
 (segment (start 123.19 121.285) (end 125.73 121.285) (width 0.25) (layer F.Cu) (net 5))
 (segment (start 125.73 135.89) (end 128.905 139.065) (width 0.25) (layer F.Cu) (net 5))
 (segment (start 125.73 121.285) (end 125.73 135.89) (width 0.25) (layer F.Cu) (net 5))
 (segment (start 128.905 139.065) (end 129.34 139.065) (width 0.25) (layer F.Cu) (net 5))
 (segment (start 129.34 139.065) (end 135.275 139.065) (width 0.25) (layer F.Cu) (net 5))
 (segment (start 123.19 128.905) (end 121.92 127.635) (width 0.25) (layer B.Cu) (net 6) (status 80000))
 (segment (start 121.92 127.635) (end 121.92 127) (width 0.25) (layer B.Cu) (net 6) (status 80000))
 (segment (start 121.92 127) (end 114.935 120.015) (width 0.25) (layer B.Cu) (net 6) (status 80000))
 (segment (start 114.935 120.015) (end 113.03 120.015) (width 0.25) (layer B.Cu) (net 6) (status 80000))
 (via (at 113.03 120.015) (size 0.6) (layers F.Cu B.Cu) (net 6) (status 80000))
 (segment (start 113.03 120.015) (end 107.315 114.3) (width 0.25) (layer F.Cu) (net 6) (status 80000))
 (segment (start 107.315 114.3) (end 107.315 108.585) (width 0.25) (layer F.Cu) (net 6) (status 80000))
 (segment (start 107.315 108.585) (end 106.045 107.315) (width 0.25) (layer F.Cu) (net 6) (status 80000))
 (segment (start 106.045 109.855) (end 107.315 111.125) (width 0.25) (layer B.Cu) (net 7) (status 80000))
 (segment (start 107.315 111.125) (end 109.22 111.125) (width 0.25) (layer B.Cu) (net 7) (status 80000))
 (via (at 109.22 111.125) (size 0.6) (layers F.Cu B.Cu) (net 7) (status 80000))
 (segment (start 109.22 111.125) (end 111.125 113.03) (width 0.25) (layer F.Cu) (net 7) (status 80000))
 (segment (start 111.125 113.03) (end 113.665 113.03) (width 0.25) (layer F.Cu) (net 7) (status 80000))
 (segment (start 113.665 113.03) (end 115.57 114.935) (width 0.25) (layer F.Cu) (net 7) (status 80000))
 (segment (start 115.57 114.935) (end 115.57 116.205) (width 0.25) (layer F.Cu) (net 7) (status 80000))
 (segment (start 115.57 116.205) (end 116.205 116.205) (width 0.25) (layer F.Cu) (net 7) (status 80000))
 (segment (start 116.205 116.205) (end 117.475 117.475) (width 0.25) (layer F.Cu) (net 7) (status 80000))
 (segment (start 117.475 117.475) (end 118.11 117.475) (width 0.25) (layer F.Cu) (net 7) (status 80000))
 (segment (start 118.11 117.475) (end 118.11 120.015) (width 0.25) (layer F.Cu) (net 7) (status 80000))
 (segment (start 118.11 120.015) (end 118.745 120.65) (width 0.25) (layer F.Cu) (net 7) (status 80000))
 (segment (start 118.745 120.65) (end 118.745 123.825) (width 0.25) (layer F.Cu) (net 7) (status 80000))
 (segment (start 118.745 123.825) (end 119.38 123.825) (width 0.25) (layer F.Cu) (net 7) (status 80000))
 (segment (start 119.38 123.825) (end 119.38 124.46) (width 0.25) (layer F.Cu) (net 7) (status 80000))
 (segment (start 119.38 124.46) (end 121.92 127) (width 0.25) (layer F.Cu) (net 7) (status 80000))
 (segment (start 121.92 127) (end 121.92 130.175) (width 0.25) (layer F.Cu) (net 7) (status 80000))
 (segment (start 121.92 130.175) (end 123.19 131.445) (width 0.25) (layer F.Cu) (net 7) (status 80000))
 (segment (start 112.395 99.06) (end 116.125 99.06) (width 0.25) (layer F.Cu) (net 8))
 (segment (start 116.125 99.06) (end 116.76 99.695) (width 0.25) (layer F.Cu) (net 8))
 (segment (start 112.395 101.6) (end 114.855 101.6) (width 0.25) (layer F.Cu) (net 9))
 (segment (start 114.855 101.6) (end 116.76 103.505) (width 0.25) (layer F.Cu) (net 9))
 (segment (start 112.395 104.14) (end 113.585 104.14) (width 0.25) (layer F.Cu) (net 10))
 (segment (start 113.585 104.14) (end 116.76 107.315) (width 0.25) (layer F.Cu) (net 10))
 (segment (start 116.76 111.125) (end 116.76 111.045) (width 0.25) (layer F.Cu) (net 11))
 (segment (start 116.76 111.045) (end 112.395 106.68) (width 0.25) (layer F.Cu) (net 11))
 (segment (start 116.76 114.935) (end 116.76 113.585) (width 0.25) (layer F.Cu) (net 12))
 (segment (start 116.76 113.585) (end 112.395 109.22) (width 0.25) (layer F.Cu) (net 12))
 (segment (start 112.395 114.3) (end 112.395 114.38) (width 0.25) (layer F.Cu) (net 13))
 (segment (start 112.395 114.38) (end 116.76 118.745) (width 0.25) (layer F.Cu) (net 13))
 (segment (start 135.89 100.965) (end 134.62 99.695) (width 0.25) (layer B.Cu) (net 16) (status 80000))
 (segment (start 134.62 99.695) (end 129.54 99.695) (width 0.25) (layer B.Cu) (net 16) (status 80000))
 (segment (start 129.54 99.695) (end 128.27 100.965) (width 0.25) (layer B.Cu) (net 16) (status 80000))
 (segment (start 128.27 100.965) (end 123.19 100.965) (width 0.25) (layer B.Cu) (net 16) (status 80000))
 (segment (start 135.89 117.475) (end 137.16 118.745) (width 0.25) (layer B.Cu) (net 18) (status 80000))
 (segment (start 137.16 118.745) (end 137.16 121.285) (width 0.25) (layer B.Cu) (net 18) (status 80000))
 (segment (start 137.16 121.285) (end 134.62 121.285) (width 0.25) (layer B.Cu) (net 18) (status 80000))
 (segment (start 134.62 121.285) (end 134.62 120.65) (width 0.25) (layer B.Cu) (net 18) (status 80000))
 (segment (start 134.62 120.65) (end 132.08 118.11) (width 0.25) (layer B.Cu) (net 18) (status 80000))
 (segment (start 132.08 118.11) (end 132.08 117.475) (width 0.25) (layer B.Cu) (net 18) (status 80000))
 (segment (start 132.08 117.475) (end 129.54 117.475) (width 0.25) (layer B.Cu) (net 18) (status 80000))
 (segment (start 129.54 117.475) (end 128.905 116.84) (width 0.25) (layer B.Cu) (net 18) (status 80000))
 (segment (start 128.905 116.84) (end 127.635 116.84) (width 0.25) (layer B.Cu) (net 18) (status 80000))
 (segment (start 127.635 116.84) (end 127.635 116.205) (width 0.25) (layer B.Cu) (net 18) (status 80000))
 (segment (start 127.635 116.205) (end 127 116.205) (width 0.25) (layer B.Cu) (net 18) (status 80000))
 (segment (start 127 116.205) (end 127 111.76) (width 0.25) (layer B.Cu) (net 18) (status 80000))
 (segment (start 127 111.76) (end 126.365 111.125) (width 0.25) (layer B.Cu) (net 18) (status 80000))
 (via (at 126.365 111.125) (size 0.6) (layers F.Cu B.Cu) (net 18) (status 80000))
 (segment (start 126.365 111.125) (end 126.365 103.505) (width 0.25) (layer F.Cu) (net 18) (status 80000))
 (via (at 126.365 103.505) (size 0.6) (layers F.Cu B.Cu) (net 18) (status 80000))
 (segment (start 126.365 103.505) (end 123.19 103.505) (width 0.25) (layer B.Cu) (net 18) (status 80000))
 (segment (start 135.89 131.445) (end 132.08 127.635) (width 0.25) (layer B.Cu) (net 20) (status 80000))
 (segment (start 132.08 127.635) (end 132.08 120.015) (width 0.25) (layer B.Cu) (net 20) (status 80000))
 (segment (start 132.08 120.015) (end 129.54 120.015) (width 0.25) (layer B.Cu) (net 20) (status 80000))
 (segment (start 129.54 120.015) (end 124.46 114.935) (width 0.25) (layer B.Cu) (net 20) (status 80000))
 (segment (start 124.46 114.935) (end 124.46 107.315) (width 0.25) (layer B.Cu) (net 20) (status 80000))
 (segment (start 124.46 107.315) (end 123.19 106.045) (width 0.25) (layer B.Cu) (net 20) (status 80000))
 (segment (start 135.89 114.935) (end 132.08 118.745) (width 0.25) (layer F.Cu) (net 21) (status 80000))
 (segment (start 132.08 118.745) (end 132.08 120.015) (width 0.25) (layer F.Cu) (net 21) (status 80000))
 (segment (start 132.08 120.015) (end 129.54 120.015) (width 0.25) (layer F.Cu) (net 21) (status 80000))
 (segment (start 129.54 120.015) (end 129.54 122.555) (width 0.25) (layer F.Cu) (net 21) (status 80000))
 (segment (start 129.54 122.555) (end 130.81 123.825) (width 0.25) (layer F.Cu) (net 21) (status 80000))
 (segment (start 135.89 114.935) (end 135.89 111.125) (width 0.25) (layer B.Cu) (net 21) (status 80000))
 (segment (start 135.89 111.125) (end 137.16 109.855) (width 0.25) (layer B.Cu) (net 21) (status 80000))
 (segment (start 137.16 109.855) (end 137.16 99.695) (width 0.25) (layer B.Cu) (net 21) (status 80000))
 (segment (start 137.16 99.695) (end 135.89 98.425) (width 0.25) (layer B.Cu) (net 21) (status 80000))
 (segment (start 123.19 108.585) (end 125.095 108.585) (width 0.25) (layer F.Cu) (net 22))
 (segment (start 125.095 99.695) (end 119.46 99.695) (width 0.25) (layer F.Cu) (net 22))
 (segment (start 125.095 108.585) (end 125.095 99.695) (width 0.25) (layer F.Cu) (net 22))
 (segment (start 135.89 120.015) (end 134.62 118.745) (width 0.25) (layer B.Cu) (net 23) (status 80000))
 (segment (start 134.62 118.745) (end 134.62 104.775) (width 0.25) (layer B.Cu) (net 23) (status 80000))
 (segment (start 134.62 104.775) (end 135.89 103.505) (width 0.25) (layer B.Cu) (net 23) (status 80000))
 (segment (start 130.81 121.285) (end 134.62 121.285) (width 0.25) (layer F.Cu) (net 23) (status 80000))
 (segment (start 134.62 121.285) (end 135.89 120.015) (width 0.25) (layer F.Cu) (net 23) (status 80000))
 (segment (start 119.46 103.505) (end 121.285 103.505) (width 0.25) (layer F.Cu) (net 24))
 (segment (start 121.285 111.125) (end 123.19 111.125) (width 0.25) (layer F.Cu) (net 24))
 (segment (start 121.285 103.505) (end 121.285 111.125) (width 0.25) (layer F.Cu) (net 24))
 (segment (start 130.81 111.125) (end 129.54 112.395) (width 0.25) (layer F.Cu) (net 27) (status 80000))
 (segment (start 129.54 112.395) (end 121.92 112.395) (width 0.25) (layer F.Cu) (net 27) (status 80000))
 (segment (start 121.92 112.395) (end 121.285 111.76) (width 0.25) (layer F.Cu) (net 27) (status 80000))
 (segment (start 121.285 111.76) (end 120.65 111.76) (width 0.25) (layer F.Cu) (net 27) (status 80000))
 (segment (start 120.65 111.76) (end 120.015 111.125) (width 0.25) (layer F.Cu) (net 27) (status 80000))
 (segment (start 120.015 111.125) (end 119.46 111.125) (width 0.25) (layer F.Cu) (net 27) (status 80000))
 (segment (start 119.46 114.935) (end 119.38 114.935) (width 0.25) (layer F.Cu) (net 28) (status 80000))
 (segment (start 119.38 114.935) (end 120.015 115.57) (width 0.25) (layer F.Cu) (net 28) (status 80000))
 (segment (start 120.015 115.57) (end 120.65 115.57) (width 0.25) (layer F.Cu) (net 28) (status 80000))
 (segment (start 120.65 115.57) (end 121.92 116.84) (width 0.25) (layer F.Cu) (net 28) (status 80000))
 (segment (start 121.92 116.84) (end 121.92 117.475) (width 0.25) (layer F.Cu) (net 28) (status 80000))
 (segment (start 121.92 117.475) (end 125.73 117.475) (width 0.25) (layer F.Cu) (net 28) (status 80000))
 (segment (start 125.73 117.475) (end 127.635 115.57) (width 0.25) (layer F.Cu) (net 28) (status 80000))
 (segment (start 127.635 115.57) (end 128.27 115.57) (width 0.25) (layer F.Cu) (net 28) (status 80000))
 (via (at 128.27 115.57) (size 0.6) (layers F.Cu B.Cu) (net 28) (status 80000))
 (segment (start 128.27 115.57) (end 129.54 114.3) (width 0.25) (layer B.Cu) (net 28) (status 80000))
 (segment (start 129.54 114.3) (end 129.54 109.855) (width 0.25) (layer B.Cu) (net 28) (status 80000))
 (segment (start 129.54 109.855) (end 130.81 108.585) (width 0.25) (layer B.Cu) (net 28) (status 80000))
 (segment (start 123.19 123.825) (end 120.65 121.285) (width 0.25) (layer F.Cu) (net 29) (status 80000))
 (segment (start 120.65 121.285) (end 120.65 117.475) (width 0.25) (layer F.Cu) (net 29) (status 80000))
 (segment (start 120.65 117.475) (end 119.38 116.205) (width 0.25) (layer F.Cu) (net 29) (status 80000))
 (segment (start 119.38 116.205) (end 118.11 116.205) (width 0.25) (layer F.Cu) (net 29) (status 80000))
 (segment (start 118.11 116.205) (end 118.11 109.855) (width 0.25) (layer F.Cu) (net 29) (status 80000))
 (segment (start 118.11 109.855) (end 119.38 108.585) (width 0.25) (layer F.Cu) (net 29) (status 80000))
 (segment (start 119.38 108.585) (end 119.38 107.315) (width 0.25) (layer F.Cu) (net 29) (status 80000))
 (segment (start 119.38 107.315) (end 119.46 107.315) (width 0.25) (layer F.Cu) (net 29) (status 80000))
 (segment (start 119.46 118.745) (end 119.46 122.635) (width 0.25) (layer F.Cu) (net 31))
 (segment (start 119.46 122.635) (end 123.19 126.365) (width 0.25) (layer F.Cu) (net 31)))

